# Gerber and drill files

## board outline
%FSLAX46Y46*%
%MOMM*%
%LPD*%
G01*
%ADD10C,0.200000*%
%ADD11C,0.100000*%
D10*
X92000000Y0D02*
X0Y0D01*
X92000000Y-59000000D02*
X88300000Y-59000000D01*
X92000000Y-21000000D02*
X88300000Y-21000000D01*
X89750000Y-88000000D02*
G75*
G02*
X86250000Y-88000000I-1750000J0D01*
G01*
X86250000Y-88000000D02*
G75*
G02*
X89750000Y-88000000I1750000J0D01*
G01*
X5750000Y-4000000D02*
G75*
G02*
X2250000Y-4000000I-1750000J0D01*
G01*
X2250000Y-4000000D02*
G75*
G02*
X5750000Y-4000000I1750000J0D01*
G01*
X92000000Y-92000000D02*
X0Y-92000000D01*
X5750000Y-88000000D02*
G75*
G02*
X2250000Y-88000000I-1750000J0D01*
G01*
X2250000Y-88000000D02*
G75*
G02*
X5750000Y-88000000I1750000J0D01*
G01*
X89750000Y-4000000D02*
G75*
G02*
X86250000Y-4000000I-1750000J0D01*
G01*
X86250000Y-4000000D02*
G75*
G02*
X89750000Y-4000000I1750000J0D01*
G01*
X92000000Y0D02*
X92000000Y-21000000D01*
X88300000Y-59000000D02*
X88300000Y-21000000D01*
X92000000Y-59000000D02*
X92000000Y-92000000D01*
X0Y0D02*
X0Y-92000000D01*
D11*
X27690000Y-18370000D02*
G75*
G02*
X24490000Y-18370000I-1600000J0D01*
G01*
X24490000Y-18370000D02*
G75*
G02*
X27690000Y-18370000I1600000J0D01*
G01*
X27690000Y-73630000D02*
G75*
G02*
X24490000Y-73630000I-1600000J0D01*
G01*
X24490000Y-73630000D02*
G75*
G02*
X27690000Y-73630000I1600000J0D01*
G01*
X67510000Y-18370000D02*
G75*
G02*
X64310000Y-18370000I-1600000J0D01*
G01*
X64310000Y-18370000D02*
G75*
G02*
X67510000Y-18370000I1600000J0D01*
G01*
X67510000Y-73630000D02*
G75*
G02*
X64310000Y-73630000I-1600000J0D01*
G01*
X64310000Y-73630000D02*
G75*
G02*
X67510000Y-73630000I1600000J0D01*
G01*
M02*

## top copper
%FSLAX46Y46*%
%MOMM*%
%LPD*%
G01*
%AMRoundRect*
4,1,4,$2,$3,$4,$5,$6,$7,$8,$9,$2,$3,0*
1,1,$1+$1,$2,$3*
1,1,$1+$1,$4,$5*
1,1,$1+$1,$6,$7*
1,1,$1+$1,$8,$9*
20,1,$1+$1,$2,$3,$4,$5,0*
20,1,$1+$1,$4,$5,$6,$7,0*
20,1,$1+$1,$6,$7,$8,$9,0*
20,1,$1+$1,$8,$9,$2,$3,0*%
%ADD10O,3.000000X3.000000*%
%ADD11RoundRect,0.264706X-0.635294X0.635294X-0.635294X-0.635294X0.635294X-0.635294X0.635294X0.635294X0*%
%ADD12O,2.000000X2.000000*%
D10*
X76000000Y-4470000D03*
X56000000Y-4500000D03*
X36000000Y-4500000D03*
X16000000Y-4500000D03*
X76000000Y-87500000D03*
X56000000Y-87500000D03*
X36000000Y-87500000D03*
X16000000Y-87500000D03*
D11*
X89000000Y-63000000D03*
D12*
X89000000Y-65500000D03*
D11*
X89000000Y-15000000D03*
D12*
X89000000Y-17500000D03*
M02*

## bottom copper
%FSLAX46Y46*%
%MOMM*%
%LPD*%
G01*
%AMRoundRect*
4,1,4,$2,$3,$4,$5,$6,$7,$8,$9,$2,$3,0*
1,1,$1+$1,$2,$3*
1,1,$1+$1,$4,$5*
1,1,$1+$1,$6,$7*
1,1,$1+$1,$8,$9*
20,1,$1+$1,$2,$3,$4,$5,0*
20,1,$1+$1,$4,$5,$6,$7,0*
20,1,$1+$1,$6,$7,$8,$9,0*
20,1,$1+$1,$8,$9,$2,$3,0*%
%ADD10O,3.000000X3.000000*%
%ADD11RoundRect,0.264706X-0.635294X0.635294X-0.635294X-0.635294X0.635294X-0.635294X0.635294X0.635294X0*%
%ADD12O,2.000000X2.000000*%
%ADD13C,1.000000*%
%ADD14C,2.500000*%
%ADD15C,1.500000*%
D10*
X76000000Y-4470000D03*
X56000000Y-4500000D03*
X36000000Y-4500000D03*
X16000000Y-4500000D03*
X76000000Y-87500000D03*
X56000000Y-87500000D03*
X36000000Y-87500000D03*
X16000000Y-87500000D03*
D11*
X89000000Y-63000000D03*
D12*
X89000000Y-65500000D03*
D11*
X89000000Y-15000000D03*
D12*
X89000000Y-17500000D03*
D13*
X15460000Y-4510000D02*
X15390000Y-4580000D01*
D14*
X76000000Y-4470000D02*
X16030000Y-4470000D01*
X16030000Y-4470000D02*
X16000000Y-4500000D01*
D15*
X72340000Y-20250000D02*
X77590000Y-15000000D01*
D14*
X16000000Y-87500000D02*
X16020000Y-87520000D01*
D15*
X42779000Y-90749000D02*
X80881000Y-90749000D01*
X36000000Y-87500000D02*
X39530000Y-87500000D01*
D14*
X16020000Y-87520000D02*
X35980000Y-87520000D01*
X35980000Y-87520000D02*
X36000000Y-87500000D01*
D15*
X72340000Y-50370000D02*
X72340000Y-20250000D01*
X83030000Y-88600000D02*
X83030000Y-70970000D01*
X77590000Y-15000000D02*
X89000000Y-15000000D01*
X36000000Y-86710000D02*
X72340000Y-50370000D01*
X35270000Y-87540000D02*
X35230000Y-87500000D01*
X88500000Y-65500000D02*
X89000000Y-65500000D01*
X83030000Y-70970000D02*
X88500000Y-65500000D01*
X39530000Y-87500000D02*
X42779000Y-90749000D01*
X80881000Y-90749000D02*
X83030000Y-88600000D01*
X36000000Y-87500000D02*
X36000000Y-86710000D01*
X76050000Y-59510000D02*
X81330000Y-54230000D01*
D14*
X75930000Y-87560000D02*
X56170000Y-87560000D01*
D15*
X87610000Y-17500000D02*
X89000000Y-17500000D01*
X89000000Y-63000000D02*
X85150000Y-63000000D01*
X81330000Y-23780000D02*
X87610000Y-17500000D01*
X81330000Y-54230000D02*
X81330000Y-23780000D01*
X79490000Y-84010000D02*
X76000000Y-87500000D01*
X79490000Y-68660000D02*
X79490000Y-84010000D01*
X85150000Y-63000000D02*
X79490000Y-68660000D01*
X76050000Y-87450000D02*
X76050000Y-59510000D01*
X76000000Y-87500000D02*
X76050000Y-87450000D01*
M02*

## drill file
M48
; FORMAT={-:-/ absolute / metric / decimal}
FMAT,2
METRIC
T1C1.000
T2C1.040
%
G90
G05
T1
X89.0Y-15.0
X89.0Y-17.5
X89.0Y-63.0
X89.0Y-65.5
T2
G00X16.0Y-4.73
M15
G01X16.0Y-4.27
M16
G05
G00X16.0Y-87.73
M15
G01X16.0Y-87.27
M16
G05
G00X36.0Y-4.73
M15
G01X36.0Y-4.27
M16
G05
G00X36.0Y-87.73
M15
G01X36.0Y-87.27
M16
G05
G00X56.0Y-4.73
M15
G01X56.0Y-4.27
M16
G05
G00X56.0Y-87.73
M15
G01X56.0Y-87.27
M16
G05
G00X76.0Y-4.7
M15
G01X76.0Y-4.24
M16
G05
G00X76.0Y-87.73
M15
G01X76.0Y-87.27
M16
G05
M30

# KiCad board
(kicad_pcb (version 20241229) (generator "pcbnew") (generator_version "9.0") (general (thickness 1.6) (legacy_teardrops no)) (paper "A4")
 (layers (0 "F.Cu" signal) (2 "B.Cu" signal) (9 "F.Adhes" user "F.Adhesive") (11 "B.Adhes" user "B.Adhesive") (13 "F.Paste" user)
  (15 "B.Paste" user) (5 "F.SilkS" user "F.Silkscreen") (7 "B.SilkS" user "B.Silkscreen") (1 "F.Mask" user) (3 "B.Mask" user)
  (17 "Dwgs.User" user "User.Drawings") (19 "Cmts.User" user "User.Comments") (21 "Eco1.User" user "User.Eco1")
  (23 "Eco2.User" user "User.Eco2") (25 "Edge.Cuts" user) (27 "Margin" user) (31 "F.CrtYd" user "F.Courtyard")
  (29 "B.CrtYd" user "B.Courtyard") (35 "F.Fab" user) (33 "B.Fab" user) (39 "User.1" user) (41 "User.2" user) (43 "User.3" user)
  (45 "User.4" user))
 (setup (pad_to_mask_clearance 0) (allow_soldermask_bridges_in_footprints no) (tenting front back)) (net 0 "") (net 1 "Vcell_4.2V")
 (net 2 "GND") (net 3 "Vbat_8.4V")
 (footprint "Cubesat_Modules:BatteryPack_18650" (layer "B.Cu") (at 46 46 180)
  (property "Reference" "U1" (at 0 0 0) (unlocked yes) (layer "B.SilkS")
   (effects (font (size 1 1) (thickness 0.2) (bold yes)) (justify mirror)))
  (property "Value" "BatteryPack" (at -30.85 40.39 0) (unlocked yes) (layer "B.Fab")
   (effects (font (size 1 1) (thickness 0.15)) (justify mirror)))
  (fp_circle (center 19.91 27.63) (end 21.51 27.63) (stroke (width 0.1) (type solid)) (fill no) (layer "Edge.Cuts"))
  (fp_circle (center 19.91 -27.63) (end 21.51 -27.63) (stroke (width 0.1) (type solid)) (fill no) (layer "Edge.Cuts"))
  (fp_circle (center -19.91 27.63) (end -18.31 27.63) (stroke (width 0.1) (type solid)) (fill no) (layer "Edge.Cuts"))
  (fp_circle (center -19.91 -27.63) (end -18.31 -27.63) (stroke (width 0.1) (type solid)) (fill no) (layer "Edge.Cuts"))
  (pad "1" thru_hole oval (at -30 41.53 90) (size 3 3) (drill oval 1.5 1.04) (layers "*.Cu" "*.Mask") (remove_unused_layers no)
   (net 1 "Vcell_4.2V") (solder_mask_margin 0.102))
  (pad "2" thru_hole oval (at -10 41.5 90) (size 3 3) (drill oval 1.5 1.04) (layers "*.Cu" "*.Mask") (remove_unused_layers no)
   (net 1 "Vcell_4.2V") (solder_mask_margin 0.102))
  (pad "3" thru_hole oval (at 10 41.5 90) (size 3 3) (drill oval 1.5 1.04) (layers "*.Cu" "*.Mask") (remove_unused_layers no)
   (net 1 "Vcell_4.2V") (solder_mask_margin 0.102))
  (pad "4" thru_hole oval (at 30 41.5 90) (size 3 3) (drill oval 1.5 1.04) (layers "*.Cu" "*.Mask") (remove_unused_layers no)
   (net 1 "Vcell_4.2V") (solder_mask_margin 0.102))
  (pad "5" thru_hole oval (at -30 -41.5 90) (size 3 3) (drill oval 1.5 1.04) (layers "*.Cu" "*.Mask") (remove_unused_layers no)
   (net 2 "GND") (solder_mask_margin 0.102))
  (pad "6" thru_hole oval (at -10 -41.5 90) (size 3 3) (drill oval 1.5 1.04) (layers "*.Cu" "*.Mask") (remove_unused_layers no)
   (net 2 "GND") (solder_mask_margin 0.102))
  (pad "7" thru_hole oval (at 10 -41.5 90) (size 3 3) (drill oval 1.5 1.04) (layers "*.Cu" "*.Mask") (remove_unused_layers no)
   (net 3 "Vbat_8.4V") (solder_mask_margin 0.102))
  (pad "8" thru_hole oval (at 30 -41.5 90) (size 3 3) (drill oval 1.5 1.04) (layers "*.Cu" "*.Mask") (remove_unused_layers no)
   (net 3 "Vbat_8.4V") (solder_mask_margin 0.102)))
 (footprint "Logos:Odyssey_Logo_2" (layer "B.Cu") (at 2.245376 55.921622 -90)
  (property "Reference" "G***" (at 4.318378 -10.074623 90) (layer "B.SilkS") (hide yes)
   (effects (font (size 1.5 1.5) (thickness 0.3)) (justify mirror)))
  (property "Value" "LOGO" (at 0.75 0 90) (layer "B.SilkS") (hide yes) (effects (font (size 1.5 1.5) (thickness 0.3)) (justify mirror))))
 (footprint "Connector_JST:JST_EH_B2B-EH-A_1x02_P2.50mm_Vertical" (layer "B.Cu") (at 89 63 -90)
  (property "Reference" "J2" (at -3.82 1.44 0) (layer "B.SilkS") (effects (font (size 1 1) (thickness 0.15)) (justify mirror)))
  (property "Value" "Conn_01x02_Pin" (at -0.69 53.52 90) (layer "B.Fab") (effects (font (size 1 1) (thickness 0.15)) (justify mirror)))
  (pad "1" thru_hole roundrect (at 0 0 270) (size 1.8 1.8) (drill 1) (layers "*.Cu" "*.Mask") (remove_unused_layers no)
   (roundrect_rratio 0.147059) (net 2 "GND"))
  (pad "2" thru_hole oval (at 2.5 0 270) (size 2 2) (drill 1) (layers "*.Cu" "*.Mask") (remove_unused_layers no) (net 3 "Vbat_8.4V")))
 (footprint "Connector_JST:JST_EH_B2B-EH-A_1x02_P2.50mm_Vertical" (layer "B.Cu") (at 89 15 -90)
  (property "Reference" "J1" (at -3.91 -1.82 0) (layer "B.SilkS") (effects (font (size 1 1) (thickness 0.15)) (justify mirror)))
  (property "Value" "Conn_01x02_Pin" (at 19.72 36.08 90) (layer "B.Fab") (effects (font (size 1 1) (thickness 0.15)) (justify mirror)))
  (pad "1" thru_hole roundrect (at 0 0 270) (size 1.8 1.8) (drill 1) (layers "*.Cu" "*.Mask") (remove_unused_layers no)
   (roundrect_rratio 0.147059) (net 3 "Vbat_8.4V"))
  (pad "2" thru_hole oval (at 2.5 0 270) (size 2 2) (drill 1) (layers "*.Cu" "*.Mask") (remove_unused_layers no) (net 2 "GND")))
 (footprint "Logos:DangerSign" (layer "B.Cu") (at 67.03 3.89 180)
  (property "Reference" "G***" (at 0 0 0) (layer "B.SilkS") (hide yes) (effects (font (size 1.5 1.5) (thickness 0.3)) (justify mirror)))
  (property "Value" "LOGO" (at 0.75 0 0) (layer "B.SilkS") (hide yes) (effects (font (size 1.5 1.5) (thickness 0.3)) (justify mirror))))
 (gr_line (start 92 0) (end 0 0) (stroke (width 0.2) (type solid)) (layer "Edge.Cuts"))
 (gr_line (start 92 59) (end 88.3 59) (stroke (width 0.2) (type solid)) (layer "Edge.Cuts"))
 (gr_line (start 92 21) (end 88.3 21) (stroke (width 0.2) (type solid)) (layer "Edge.Cuts"))
 (gr_circle (center 88 88) (end 86.25 88) (stroke (width 0.2) (type solid)) (fill no) (layer "Edge.Cuts"))
 (gr_circle (center 4 4) (end 2.25 4) (stroke (width 0.2) (type solid)) (fill no) (layer "Edge.Cuts"))
 (gr_line (start 92 92) (end 0 92) (stroke (width 0.2) (type solid)) (layer "Edge.Cuts"))
 (gr_circle (center 4 88) (end 2.25 88) (stroke (width 0.2) (type solid)) (fill no) (layer "Edge.Cuts"))
 (gr_circle (center 88 4) (end 86.25 4) (stroke (width 0.2) (type solid)) (fill no) (layer "Edge.Cuts"))
 (gr_line (start 92 0) (end 92 21) (stroke (width 0.2) (type solid)) (layer "Edge.Cuts"))
 (gr_line (start 88.3 59) (end 88.3 21) (stroke (width 0.2) (type solid)) (layer "Edge.Cuts"))
 (gr_line (start 92 59) (end 92 92) (stroke (width 0.2) (type solid)) (layer "Edge.Cuts"))
 (gr_line (start 0 0) (end 0 92) (stroke (width 0.2) (type solid)) (layer "Edge.Cuts"))
 (segment (start 15.46 4.51) (end 15.39 4.58) (width 1) (layer "B.Cu") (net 1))
 (segment (start 76 4.47) (end 16.03 4.47) (width 2.5) (layer "B.Cu") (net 1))
 (segment (start 16.03 4.47) (end 16 4.5) (width 2.5) (layer "B.Cu") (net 1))
 (segment (start 72.34 20.25) (end 77.59 15) (width 1.5) (layer "B.Cu") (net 3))
 (segment (start 16 87.5) (end 16.02 87.52) (width 2.5) (layer "B.Cu") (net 3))
 (segment (start 42.779 90.749) (end 80.881 90.749) (width 1.5) (layer "B.Cu") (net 3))
 (segment (start 36 87.5) (end 39.53 87.5) (width 1.5) (layer "B.Cu") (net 3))
 (segment (start 16.02 87.52) (end 35.98 87.52) (width 2.5) (layer "B.Cu") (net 3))
 (segment (start 35.98 87.52) (end 36 87.5) (width 2.5) (layer "B.Cu") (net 3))
 (segment (start 72.34 50.37) (end 72.34 20.25) (width 1.5) (layer "B.Cu") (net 3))
 (segment (start 83.03 88.6) (end 83.03 70.97) (width 1.5) (layer "B.Cu") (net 3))
 (segment (start 77.59 15) (end 89 15) (width 1.5) (layer "B.Cu") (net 3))
 (segment (start 36 86.71) (end 72.34 50.37) (width 1.5) (layer "B.Cu") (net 3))
 (segment (start 35.27 87.54) (end 35.23 87.5) (width 1.5) (layer "B.Cu") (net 3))
 (segment (start 88.5 65.5) (end 89 65.5) (width 1.5) (layer "B.Cu") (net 3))
 (segment (start 83.03 70.97) (end 88.5 65.5) (width 1.5) (layer "B.Cu") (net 3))
 (segment (start 39.53 87.5) (end 42.779 90.749) (width 1.5) (layer "B.Cu") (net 3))
 (segment (start 80.881 90.749) (end 83.03 88.6) (width 1.5) (layer "B.Cu") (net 3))
 (segment (start 36 87.5) (end 36 86.71) (width 1.5) (layer "B.Cu") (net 3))
 (segment (start 76.05 59.51) (end 81.33 54.23) (width 1.5) (layer "B.Cu") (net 2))
 (segment (start 75.93 87.56) (end 56.17 87.56) (width 2.5) (layer "B.Cu") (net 2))
 (segment (start 87.61 17.5) (end 89 17.5) (width 1.5) (layer "B.Cu") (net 2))
 (segment (start 89 63) (end 85.15 63) (width 1.5) (layer "B.Cu") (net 2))
 (segment (start 81.33 23.78) (end 87.61 17.5) (width 1.5) (layer "B.Cu") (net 2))
 (segment (start 81.33 54.23) (end 81.33 23.78) (width 1.5) (layer "B.Cu") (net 2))
 (segment (start 79.49 84.01) (end 76 87.5) (width 1.5) (layer "B.Cu") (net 2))
 (segment (start 79.49 68.66) (end 79.49 84.01) (width 1.5) (layer "B.Cu") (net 2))
 (segment (start 85.15 63) (end 79.49 68.66) (width 1.5) (layer "B.Cu") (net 2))
 (segment (start 76.05 87.45) (end 76.05 59.51) (width 1.5) (layer "B.Cu") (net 2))
 (segment (start 76 87.5) (end 76.05 87.45) (width 1.5) (layer "B.Cu") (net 2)))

